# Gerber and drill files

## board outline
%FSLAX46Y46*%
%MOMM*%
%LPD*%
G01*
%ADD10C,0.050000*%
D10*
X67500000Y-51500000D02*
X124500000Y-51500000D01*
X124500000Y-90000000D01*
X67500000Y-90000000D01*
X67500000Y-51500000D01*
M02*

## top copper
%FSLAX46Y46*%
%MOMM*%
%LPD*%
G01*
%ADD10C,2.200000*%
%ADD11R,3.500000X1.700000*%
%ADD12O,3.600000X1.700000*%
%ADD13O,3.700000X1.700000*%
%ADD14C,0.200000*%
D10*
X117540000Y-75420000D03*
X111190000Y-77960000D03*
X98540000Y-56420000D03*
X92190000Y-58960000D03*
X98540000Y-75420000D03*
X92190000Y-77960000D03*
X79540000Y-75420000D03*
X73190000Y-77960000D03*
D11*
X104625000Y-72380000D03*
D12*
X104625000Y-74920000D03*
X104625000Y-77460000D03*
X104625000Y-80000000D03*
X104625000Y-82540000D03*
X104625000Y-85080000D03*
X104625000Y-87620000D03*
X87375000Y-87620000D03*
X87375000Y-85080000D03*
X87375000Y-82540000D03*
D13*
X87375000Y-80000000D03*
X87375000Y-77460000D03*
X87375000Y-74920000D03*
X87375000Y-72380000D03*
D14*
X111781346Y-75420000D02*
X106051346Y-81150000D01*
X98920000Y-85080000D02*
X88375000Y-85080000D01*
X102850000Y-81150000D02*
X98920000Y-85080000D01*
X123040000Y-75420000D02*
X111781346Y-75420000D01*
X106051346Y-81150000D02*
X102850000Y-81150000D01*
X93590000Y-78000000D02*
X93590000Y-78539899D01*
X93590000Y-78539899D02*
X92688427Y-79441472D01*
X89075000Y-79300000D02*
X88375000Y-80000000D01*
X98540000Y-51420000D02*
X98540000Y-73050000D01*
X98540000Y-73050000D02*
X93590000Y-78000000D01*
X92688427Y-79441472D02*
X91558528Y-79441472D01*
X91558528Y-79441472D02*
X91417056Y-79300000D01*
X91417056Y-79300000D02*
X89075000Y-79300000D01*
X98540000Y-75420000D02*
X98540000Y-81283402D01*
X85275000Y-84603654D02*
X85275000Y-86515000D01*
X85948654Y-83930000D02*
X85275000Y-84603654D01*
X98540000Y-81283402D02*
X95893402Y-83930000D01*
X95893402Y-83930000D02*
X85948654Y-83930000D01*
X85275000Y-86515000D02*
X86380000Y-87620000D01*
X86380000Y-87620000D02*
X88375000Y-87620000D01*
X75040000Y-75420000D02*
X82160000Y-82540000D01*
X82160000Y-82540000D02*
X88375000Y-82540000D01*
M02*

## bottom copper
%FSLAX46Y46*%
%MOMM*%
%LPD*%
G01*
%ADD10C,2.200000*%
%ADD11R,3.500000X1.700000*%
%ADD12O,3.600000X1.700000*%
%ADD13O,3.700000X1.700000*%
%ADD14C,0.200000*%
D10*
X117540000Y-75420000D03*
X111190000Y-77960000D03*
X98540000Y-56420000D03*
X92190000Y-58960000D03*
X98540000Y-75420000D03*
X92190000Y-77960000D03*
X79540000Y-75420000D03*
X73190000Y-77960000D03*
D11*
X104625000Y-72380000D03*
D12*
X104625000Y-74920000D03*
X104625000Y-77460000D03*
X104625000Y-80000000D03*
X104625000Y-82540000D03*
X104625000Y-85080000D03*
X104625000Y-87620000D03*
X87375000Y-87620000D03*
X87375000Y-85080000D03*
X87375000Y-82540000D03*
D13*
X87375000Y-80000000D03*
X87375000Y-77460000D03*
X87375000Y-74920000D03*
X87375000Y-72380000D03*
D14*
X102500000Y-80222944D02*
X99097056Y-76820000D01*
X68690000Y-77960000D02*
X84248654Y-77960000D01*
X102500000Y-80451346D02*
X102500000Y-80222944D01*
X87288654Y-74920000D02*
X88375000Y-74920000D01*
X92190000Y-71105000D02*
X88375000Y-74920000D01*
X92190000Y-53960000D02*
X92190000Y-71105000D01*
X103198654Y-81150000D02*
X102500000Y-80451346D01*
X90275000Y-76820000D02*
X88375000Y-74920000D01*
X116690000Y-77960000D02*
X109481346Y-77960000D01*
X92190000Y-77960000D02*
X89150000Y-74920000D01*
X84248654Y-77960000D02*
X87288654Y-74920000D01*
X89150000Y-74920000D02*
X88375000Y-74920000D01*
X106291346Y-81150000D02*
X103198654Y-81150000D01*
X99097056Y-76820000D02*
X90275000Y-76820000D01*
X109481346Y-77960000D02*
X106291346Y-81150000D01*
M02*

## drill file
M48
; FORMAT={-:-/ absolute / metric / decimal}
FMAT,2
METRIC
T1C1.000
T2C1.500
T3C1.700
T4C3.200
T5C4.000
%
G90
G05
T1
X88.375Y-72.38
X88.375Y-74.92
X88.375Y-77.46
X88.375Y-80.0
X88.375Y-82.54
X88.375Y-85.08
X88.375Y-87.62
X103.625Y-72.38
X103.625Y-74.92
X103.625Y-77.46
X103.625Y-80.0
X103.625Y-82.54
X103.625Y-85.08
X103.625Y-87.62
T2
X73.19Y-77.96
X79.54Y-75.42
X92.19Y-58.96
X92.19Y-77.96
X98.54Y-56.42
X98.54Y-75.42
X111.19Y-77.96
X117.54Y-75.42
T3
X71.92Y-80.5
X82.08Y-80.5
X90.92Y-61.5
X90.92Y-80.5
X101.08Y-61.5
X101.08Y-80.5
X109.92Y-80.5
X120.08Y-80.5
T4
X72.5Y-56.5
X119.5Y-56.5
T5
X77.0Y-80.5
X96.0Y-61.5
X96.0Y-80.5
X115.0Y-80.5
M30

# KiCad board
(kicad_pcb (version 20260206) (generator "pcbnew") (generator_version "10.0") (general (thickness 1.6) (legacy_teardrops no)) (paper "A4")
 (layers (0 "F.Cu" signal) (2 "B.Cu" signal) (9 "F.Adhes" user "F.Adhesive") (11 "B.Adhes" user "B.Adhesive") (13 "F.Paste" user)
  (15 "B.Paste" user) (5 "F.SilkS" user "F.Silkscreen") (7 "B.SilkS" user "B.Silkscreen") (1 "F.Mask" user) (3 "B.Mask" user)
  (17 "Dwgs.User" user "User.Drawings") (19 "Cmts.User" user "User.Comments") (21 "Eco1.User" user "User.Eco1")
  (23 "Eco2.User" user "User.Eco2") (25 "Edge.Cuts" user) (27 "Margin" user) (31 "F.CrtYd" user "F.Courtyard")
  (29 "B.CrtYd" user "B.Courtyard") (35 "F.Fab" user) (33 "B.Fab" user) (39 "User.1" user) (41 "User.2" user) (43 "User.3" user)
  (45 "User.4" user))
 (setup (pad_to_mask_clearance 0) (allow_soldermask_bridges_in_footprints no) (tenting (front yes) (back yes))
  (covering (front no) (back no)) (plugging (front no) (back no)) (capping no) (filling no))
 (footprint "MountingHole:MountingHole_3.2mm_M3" (layer "F.Cu") (at 72.5 56.5)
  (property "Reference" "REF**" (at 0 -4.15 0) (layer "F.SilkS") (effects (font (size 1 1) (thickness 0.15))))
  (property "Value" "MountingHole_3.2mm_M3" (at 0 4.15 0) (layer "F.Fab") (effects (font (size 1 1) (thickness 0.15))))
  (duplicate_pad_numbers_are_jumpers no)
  (pad "" np_thru_hole circle (at 0 0) (size 3.2 3.2) (drill 3.2) (layers "*.Cu" "*.Mask")))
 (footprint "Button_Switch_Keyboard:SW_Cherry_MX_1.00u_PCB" (layer "F.Cu") (at 117.54 75.42)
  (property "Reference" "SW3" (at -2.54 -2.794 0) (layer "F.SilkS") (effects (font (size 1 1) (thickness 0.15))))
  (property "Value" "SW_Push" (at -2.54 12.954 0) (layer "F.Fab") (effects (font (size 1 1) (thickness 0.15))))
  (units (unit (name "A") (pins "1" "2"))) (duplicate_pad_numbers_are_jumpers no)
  (pad "" np_thru_hole circle (at -7.62 5.08) (size 1.7 1.7) (drill 1.7) (layers "*.Cu" "*.Mask"))
  (pad "" np_thru_hole circle (at -2.54 5.08) (size 4 4) (drill 4) (layers "*.Cu" "*.Mask"))
  (pad "" np_thru_hole circle (at 2.54 5.08) (size 1.7 1.7) (drill 1.7) (layers "*.Cu" "*.Mask"))
  (pad "1" thru_hole circle (at 0 0) (size 2.2 2.2) (drill 1.5) (layers "*.Cu" "*.Mask") (remove_unused_layers no)
   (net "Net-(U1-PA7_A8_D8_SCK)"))
  (pad "2" thru_hole circle (at -6.35 2.54) (size 2.2 2.2) (drill 1.5) (layers "*.Cu" "*.Mask") (remove_unused_layers no) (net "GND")))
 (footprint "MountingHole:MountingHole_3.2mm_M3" (layer "F.Cu") (at 119.5 56.5)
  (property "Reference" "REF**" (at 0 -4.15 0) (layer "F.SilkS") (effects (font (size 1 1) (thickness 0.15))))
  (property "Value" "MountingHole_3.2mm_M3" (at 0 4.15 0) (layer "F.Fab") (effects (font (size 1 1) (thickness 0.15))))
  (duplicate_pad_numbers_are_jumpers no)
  (pad "" np_thru_hole circle (at 0 0) (size 3.2 3.2) (drill 3.2) (layers "*.Cu" "*.Mask")))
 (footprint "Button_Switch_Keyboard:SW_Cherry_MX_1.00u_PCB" (layer "F.Cu") (at 98.54 56.42)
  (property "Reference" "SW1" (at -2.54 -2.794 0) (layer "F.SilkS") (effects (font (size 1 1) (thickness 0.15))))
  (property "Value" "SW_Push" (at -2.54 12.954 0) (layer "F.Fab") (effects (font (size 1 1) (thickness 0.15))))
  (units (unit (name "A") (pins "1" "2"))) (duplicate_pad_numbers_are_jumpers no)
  (pad "" np_thru_hole circle (at -7.62 5.08) (size 1.7 1.7) (drill 1.7) (layers "*.Cu" "*.Mask"))
  (pad "" np_thru_hole circle (at -2.54 5.08) (size 4 4) (drill 4) (layers "*.Cu" "*.Mask"))
  (pad "" np_thru_hole circle (at 2.54 5.08) (size 1.7 1.7) (drill 1.7) (layers "*.Cu" "*.Mask"))
  (pad "1" thru_hole circle (at 0 0) (size 2.2 2.2) (drill 1.5) (layers "*.Cu" "*.Mask") (remove_unused_layers no)
   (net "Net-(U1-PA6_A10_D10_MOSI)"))
  (pad "2" thru_hole circle (at -6.35 2.54) (size 2.2 2.2) (drill 1.5) (layers "*.Cu" "*.Mask") (remove_unused_layers no) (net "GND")))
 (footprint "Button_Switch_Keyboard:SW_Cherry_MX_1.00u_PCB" (layer "F.Cu") (at 98.54 75.42)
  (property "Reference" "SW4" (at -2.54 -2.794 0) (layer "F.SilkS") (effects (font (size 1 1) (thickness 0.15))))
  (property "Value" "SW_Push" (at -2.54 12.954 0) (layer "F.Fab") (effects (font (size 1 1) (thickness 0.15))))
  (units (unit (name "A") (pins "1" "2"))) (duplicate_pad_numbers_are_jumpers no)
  (pad "" np_thru_hole circle (at -7.62 5.08) (size 1.7 1.7) (drill 1.7) (layers "*.Cu" "*.Mask"))
  (pad "" np_thru_hole circle (at -2.54 5.08) (size 4 4) (drill 4) (layers "*.Cu" "*.Mask"))
  (pad "" np_thru_hole circle (at 2.54 5.08) (size 1.7 1.7) (drill 1.7) (layers "*.Cu" "*.Mask"))
  (pad "1" thru_hole circle (at 0 0) (size 2.2 2.2) (drill 1.5) (layers "*.Cu" "*.Mask") (remove_unused_layers no)
   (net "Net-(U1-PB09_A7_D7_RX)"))
  (pad "2" thru_hole circle (at -6.35 2.54) (size 2.2 2.2) (drill 1.5) (layers "*.Cu" "*.Mask") (remove_unused_layers no) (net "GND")))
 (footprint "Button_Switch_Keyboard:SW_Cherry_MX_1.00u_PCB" (layer "F.Cu") (at 79.54 75.42)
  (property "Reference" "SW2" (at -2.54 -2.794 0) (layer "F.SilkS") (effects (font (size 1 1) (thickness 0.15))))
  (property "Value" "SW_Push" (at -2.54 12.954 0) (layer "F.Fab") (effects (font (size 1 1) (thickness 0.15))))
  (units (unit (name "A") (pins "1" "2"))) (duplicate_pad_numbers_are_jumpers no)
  (pad "" np_thru_hole circle (at -7.62 5.08) (size 1.7 1.7) (drill 1.7) (layers "*.Cu" "*.Mask"))
  (pad "" np_thru_hole circle (at -2.54 5.08) (size 4 4) (drill 4) (layers "*.Cu" "*.Mask"))
  (pad "" np_thru_hole circle (at 2.54 5.08) (size 1.7 1.7) (drill 1.7) (layers "*.Cu" "*.Mask"))
  (pad "1" thru_hole circle (at 0 0) (size 2.2 2.2) (drill 1.5) (layers "*.Cu" "*.Mask") (remove_unused_layers no)
   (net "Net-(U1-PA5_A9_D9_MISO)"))
  (pad "2" thru_hole circle (at -6.35 2.54) (size 2.2 2.2) (drill 1.5) (layers "*.Cu" "*.Mask") (remove_unused_layers no) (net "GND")))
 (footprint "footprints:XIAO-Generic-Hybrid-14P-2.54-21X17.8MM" (layer "B.Cu") (at 96 80 180)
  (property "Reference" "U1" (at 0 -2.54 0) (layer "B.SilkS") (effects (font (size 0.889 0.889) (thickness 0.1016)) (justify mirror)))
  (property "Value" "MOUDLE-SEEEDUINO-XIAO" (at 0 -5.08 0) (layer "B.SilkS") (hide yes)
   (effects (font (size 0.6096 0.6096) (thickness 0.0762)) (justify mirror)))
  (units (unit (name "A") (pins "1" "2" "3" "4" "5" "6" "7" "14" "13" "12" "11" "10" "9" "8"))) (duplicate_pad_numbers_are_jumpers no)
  (pad "1" thru_hole rect (at -7.625 7.62 180) (size 3.5 1.7) (drill 1 (offset -1 0)) (layers "*.Cu" "*.Mask") (remove_unused_layers no)
   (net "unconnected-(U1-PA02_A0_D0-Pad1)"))
  (pad "2" thru_hole oval (at -7.625 5.08 180) (size 3.6 1.7) (drill 1 (offset -1 0)) (layers "*.Cu" "*.Mask") (remove_unused_layers no)
   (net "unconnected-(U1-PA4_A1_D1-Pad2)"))
  (pad "3" thru_hole oval (at -7.625 2.54 180) (size 3.6 1.7) (drill 1 (offset -1 0)) (layers "*.Cu" "*.Mask") (remove_unused_layers no)
   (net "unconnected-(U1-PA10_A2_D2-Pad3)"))
  (pad "4" thru_hole oval (at -7.625 0 180) (size 3.6 1.7) (drill 1 (offset -1 0)) (layers "*.Cu" "*.Mask") (remove_unused_layers no)
   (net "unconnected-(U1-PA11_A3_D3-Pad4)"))
  (pad "5" thru_hole oval (at -7.625 -2.54 180) (size 3.6 1.7) (drill 1 (offset -1 0)) (layers "*.Cu" "*.Mask") (remove_unused_layers no)
   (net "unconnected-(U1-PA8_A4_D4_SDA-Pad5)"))
  (pad "6" thru_hole oval (at -7.625 -5.08) (size 3.6 1.7) (drill 1 (offset 1 0)) (layers "*.Cu" "*.Mask") (remove_unused_layers no)
   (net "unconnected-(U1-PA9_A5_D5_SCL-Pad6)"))
  (pad "7" thru_hole oval (at -7.625 -7.62 180) (size 3.6 1.7) (drill 1 (offset -1 0)) (layers "*.Cu" "*.Mask") (remove_unused_layers no)
   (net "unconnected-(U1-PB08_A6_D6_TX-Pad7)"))
  (pad "8" thru_hole oval (at 7.625 -7.62 180) (size 3.6 1.7) (drill 1 (offset 1 0)) (layers "*.Cu" "*.Mask") (remove_unused_layers no)
   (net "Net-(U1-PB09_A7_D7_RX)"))
  (pad "9" thru_hole oval (at 7.625 -5.08 180) (size 3.6 1.7) (drill 1 (offset 1 0)) (layers "*.Cu" "*.Mask") (remove_unused_layers no)
   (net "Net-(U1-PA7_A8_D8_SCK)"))
  (pad "10" thru_hole oval (at 7.625 -2.54 180) (size 3.6 1.7) (drill 1 (offset 1 0)) (layers "*.Cu" "*.Mask") (remove_unused_layers no)
   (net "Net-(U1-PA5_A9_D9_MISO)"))
  (pad "11" thru_hole oval (at 7.625 0 180) (size 3.7 1.7) (drill 1 (offset 1 0)) (layers "*.Cu" "*.Mask") (remove_unused_layers no)
   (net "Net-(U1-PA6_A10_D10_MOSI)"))
  (pad "12" thru_hole oval (at 7.625 2.54 180) (size 3.7 1.7) (drill 1 (offset 1 0)) (layers "*.Cu" "*.Mask") (remove_unused_layers no)
   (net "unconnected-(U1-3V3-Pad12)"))
  (pad "13" thru_hole oval (at 7.625 5.08 180) (size 3.7 1.7) (drill 1 (offset 1 0)) (layers "*.Cu" "*.Mask") (remove_unused_layers no)
   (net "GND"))
  (pad "14" thru_hole oval (at 7.625 7.62 180) (size 3.7 1.7) (drill 1 (offset 1 0)) (layers "*.Cu" "*.Mask") (remove_unused_layers no)
   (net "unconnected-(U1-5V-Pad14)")))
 (gr_rect (start 67.5 51.5) (end 124.5 90) (stroke (width 0.05) (type default)) (fill no) (layer "Edge.Cuts"))
 (segment (start 111.781346 75.42) (end 106.051346 81.15) (width 0.2) (layer "F.Cu") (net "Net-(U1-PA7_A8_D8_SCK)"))
 (segment (start 98.92 85.08) (end 88.375 85.08) (width 0.2) (layer "F.Cu") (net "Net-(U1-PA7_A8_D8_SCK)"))
 (segment (start 102.85 81.15) (end 98.92 85.08) (width 0.2) (layer "F.Cu") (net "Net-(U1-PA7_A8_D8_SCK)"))
 (segment (start 123.04 75.42) (end 111.781346 75.42) (width 0.2) (layer "F.Cu") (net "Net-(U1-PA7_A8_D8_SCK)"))
 (segment (start 106.051346 81.15) (end 102.85 81.15) (width 0.2) (layer "F.Cu") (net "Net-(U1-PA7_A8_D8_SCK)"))
 (segment (start 102.5 80.222944) (end 99.097056 76.82) (width 0.2) (layer "B.Cu") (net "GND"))
 (segment (start 68.69 77.96) (end 84.248654 77.96) (width 0.2) (layer "B.Cu") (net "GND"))
 (segment (start 102.5 80.451346) (end 102.5 80.222944) (width 0.2) (layer "B.Cu") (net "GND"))
 (segment (start 87.288654 74.92) (end 88.375 74.92) (width 0.2) (layer "B.Cu") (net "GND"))
 (segment (start 92.19 71.105) (end 88.375 74.92) (width 0.2) (layer "B.Cu") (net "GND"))
 (segment (start 92.19 53.96) (end 92.19 71.105) (width 0.2) (layer "B.Cu") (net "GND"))
 (segment (start 103.198654 81.15) (end 102.5 80.451346) (width 0.2) (layer "B.Cu") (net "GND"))
 (segment (start 90.275 76.82) (end 88.375 74.92) (width 0.2) (layer "B.Cu") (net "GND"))
 (segment (start 116.69 77.96) (end 109.481346 77.96) (width 0.2) (layer "B.Cu") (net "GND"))
 (segment (start 92.19 77.96) (end 89.15 74.92) (width 0.2) (layer "B.Cu") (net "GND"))
 (segment (start 84.248654 77.96) (end 87.288654 74.92) (width 0.2) (layer "B.Cu") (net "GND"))
 (segment (start 89.15 74.92) (end 88.375 74.92) (width 0.2) (layer "B.Cu") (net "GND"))
 (segment (start 106.291346 81.15) (end 103.198654 81.15) (width 0.2) (layer "B.Cu") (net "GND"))
 (segment (start 99.097056 76.82) (end 90.275 76.82) (width 0.2) (layer "B.Cu") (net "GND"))
 (segment (start 109.481346 77.96) (end 106.291346 81.15) (width 0.2) (layer "B.Cu") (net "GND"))
 (segment (start 93.59 78) (end 93.59 78.539899) (width 0.2) (layer "F.Cu") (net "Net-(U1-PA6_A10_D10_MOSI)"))
 (segment (start 93.59 78.539899) (end 92.688427 79.441472) (width 0.2) (layer "F.Cu") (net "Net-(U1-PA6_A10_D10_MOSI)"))
 (segment (start 89.075 79.3) (end 88.375 80) (width 0.2) (layer "F.Cu") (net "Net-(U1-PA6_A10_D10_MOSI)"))
 (segment (start 98.54 51.42) (end 98.54 73.05) (width 0.2) (layer "F.Cu") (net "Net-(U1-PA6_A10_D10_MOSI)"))
 (segment (start 98.54 73.05) (end 93.59 78) (width 0.2) (layer "F.Cu") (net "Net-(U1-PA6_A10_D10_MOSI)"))
 (segment (start 92.688427 79.441472) (end 91.558528 79.441472) (width 0.2) (layer "F.Cu") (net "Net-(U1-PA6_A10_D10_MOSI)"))
 (segment (start 91.558528 79.441472) (end 91.417056 79.3) (width 0.2) (layer "F.Cu") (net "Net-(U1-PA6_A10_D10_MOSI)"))
 (segment (start 91.417056 79.3) (end 89.075 79.3) (width 0.2) (layer "F.Cu") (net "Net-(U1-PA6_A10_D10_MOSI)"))
 (segment (start 98.54 75.42) (end 98.54 81.283402) (width 0.2) (layer "F.Cu") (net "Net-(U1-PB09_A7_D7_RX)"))
 (segment (start 85.275 84.603654) (end 85.275 86.515) (width 0.2) (layer "F.Cu") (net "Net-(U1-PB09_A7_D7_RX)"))
 (segment (start 85.948654 83.93) (end 85.275 84.603654) (width 0.2) (layer "F.Cu") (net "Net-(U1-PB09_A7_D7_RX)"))
 (segment (start 98.54 81.283402) (end 95.893402 83.93) (width 0.2) (layer "F.Cu") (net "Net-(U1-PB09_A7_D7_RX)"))
 (segment (start 95.893402 83.93) (end 85.948654 83.93) (width 0.2) (layer "F.Cu") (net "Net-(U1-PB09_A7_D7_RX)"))
 (segment (start 85.275 86.515) (end 86.38 87.62) (width 0.2) (layer "F.Cu") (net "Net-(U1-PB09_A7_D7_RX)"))
 (segment (start 86.38 87.62) (end 88.375 87.62) (width 0.2) (layer "F.Cu") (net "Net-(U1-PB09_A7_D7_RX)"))
 (segment (start 75.04 75.42) (end 82.16 82.54) (width 0.2) (layer "F.Cu") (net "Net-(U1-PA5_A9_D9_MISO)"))
 (segment (start 82.16 82.54) (end 88.375 82.54) (width 0.2) (layer "F.Cu") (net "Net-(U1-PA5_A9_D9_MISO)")))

